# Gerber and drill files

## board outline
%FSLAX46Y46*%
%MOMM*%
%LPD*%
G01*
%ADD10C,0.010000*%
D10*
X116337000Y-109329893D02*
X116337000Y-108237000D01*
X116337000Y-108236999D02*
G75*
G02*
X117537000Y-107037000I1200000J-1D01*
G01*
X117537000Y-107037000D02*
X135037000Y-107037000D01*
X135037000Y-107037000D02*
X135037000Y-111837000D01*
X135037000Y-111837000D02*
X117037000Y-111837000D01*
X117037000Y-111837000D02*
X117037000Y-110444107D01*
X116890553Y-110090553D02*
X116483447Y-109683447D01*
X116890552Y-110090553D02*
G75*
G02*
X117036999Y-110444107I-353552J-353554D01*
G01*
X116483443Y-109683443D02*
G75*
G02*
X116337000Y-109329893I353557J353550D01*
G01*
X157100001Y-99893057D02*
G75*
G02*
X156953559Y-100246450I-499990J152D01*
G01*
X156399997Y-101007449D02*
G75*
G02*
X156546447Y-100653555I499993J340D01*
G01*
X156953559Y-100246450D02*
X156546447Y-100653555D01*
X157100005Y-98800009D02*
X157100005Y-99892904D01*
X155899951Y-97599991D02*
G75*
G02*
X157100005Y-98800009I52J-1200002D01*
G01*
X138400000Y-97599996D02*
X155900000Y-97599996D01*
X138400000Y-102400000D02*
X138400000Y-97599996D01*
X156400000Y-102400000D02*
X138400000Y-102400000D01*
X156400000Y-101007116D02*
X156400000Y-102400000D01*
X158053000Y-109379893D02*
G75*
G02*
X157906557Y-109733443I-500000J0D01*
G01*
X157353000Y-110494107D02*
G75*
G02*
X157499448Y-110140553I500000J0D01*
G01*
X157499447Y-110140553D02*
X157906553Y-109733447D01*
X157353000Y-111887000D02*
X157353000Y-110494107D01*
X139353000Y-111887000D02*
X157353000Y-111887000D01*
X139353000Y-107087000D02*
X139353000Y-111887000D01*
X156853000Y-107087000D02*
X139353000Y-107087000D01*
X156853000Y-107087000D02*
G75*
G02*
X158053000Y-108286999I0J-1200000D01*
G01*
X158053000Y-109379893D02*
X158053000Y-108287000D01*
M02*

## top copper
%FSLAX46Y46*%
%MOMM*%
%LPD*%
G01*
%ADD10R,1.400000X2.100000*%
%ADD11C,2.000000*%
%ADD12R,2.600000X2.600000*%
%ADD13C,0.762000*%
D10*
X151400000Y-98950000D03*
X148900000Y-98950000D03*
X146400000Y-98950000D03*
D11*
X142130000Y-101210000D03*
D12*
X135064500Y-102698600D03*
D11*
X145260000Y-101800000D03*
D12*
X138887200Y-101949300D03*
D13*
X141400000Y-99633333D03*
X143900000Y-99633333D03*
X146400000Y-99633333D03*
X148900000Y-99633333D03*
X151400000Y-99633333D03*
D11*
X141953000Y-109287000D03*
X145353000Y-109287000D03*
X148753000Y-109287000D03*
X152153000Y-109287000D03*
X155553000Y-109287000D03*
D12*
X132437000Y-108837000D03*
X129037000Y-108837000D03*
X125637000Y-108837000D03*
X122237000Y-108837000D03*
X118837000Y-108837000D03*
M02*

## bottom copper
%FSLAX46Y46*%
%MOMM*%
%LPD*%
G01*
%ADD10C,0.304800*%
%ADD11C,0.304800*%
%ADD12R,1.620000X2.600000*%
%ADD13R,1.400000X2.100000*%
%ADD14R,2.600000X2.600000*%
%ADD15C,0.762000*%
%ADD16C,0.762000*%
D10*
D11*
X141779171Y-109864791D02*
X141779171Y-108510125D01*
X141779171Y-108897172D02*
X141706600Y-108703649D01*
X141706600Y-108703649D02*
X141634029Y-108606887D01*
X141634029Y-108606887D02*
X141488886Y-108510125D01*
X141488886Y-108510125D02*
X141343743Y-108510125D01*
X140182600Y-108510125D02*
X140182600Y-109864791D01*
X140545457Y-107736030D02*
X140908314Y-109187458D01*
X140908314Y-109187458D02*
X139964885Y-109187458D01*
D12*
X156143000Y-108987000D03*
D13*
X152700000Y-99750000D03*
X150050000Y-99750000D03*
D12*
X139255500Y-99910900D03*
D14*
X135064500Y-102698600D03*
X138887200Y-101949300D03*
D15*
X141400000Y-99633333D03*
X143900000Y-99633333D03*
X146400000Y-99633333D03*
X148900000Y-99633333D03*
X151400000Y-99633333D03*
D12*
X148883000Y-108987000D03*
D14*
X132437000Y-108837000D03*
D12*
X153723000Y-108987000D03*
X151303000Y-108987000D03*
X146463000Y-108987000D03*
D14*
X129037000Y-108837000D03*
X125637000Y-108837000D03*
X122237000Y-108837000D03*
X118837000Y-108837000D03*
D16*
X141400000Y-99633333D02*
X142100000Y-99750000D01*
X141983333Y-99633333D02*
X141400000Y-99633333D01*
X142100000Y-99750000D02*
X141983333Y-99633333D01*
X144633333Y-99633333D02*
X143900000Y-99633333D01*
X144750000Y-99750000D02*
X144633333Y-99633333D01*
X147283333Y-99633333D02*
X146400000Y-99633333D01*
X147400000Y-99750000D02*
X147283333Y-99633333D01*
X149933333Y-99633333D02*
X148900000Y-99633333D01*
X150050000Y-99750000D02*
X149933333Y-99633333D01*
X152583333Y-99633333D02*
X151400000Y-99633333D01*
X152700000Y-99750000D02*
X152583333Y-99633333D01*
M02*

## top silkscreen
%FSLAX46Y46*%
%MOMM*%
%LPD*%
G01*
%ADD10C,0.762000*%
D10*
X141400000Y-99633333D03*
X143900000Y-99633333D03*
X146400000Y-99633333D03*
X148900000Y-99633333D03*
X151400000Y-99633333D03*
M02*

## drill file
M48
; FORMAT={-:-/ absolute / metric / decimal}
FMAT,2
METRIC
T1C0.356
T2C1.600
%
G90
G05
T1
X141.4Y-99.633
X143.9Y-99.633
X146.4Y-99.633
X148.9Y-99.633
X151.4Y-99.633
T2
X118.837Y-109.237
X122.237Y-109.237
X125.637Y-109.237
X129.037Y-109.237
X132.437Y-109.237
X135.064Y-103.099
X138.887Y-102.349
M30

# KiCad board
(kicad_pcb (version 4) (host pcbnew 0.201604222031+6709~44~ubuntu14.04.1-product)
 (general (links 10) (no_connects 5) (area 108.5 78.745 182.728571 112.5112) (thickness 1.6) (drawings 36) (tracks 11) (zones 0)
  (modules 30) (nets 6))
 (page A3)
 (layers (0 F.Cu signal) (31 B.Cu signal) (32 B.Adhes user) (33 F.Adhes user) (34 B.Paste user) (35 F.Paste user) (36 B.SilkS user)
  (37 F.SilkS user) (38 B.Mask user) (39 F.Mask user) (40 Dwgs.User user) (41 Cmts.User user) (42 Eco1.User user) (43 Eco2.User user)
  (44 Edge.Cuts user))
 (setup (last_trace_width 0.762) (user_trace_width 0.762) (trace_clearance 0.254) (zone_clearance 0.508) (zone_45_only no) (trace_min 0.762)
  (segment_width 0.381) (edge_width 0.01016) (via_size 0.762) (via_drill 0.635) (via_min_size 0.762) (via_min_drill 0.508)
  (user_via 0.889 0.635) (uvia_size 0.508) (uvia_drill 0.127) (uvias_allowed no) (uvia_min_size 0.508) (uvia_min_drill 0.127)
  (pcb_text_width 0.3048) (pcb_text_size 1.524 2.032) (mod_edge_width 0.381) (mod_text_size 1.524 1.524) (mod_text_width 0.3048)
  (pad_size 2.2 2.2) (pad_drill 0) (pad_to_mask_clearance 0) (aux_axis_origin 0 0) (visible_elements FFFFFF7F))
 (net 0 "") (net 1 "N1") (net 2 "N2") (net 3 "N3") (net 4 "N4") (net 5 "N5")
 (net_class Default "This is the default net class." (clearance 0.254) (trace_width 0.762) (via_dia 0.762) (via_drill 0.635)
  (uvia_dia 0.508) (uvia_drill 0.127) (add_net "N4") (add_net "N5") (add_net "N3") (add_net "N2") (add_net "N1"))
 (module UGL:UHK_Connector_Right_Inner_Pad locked (layer B.Cu) (at 156.143 108.987)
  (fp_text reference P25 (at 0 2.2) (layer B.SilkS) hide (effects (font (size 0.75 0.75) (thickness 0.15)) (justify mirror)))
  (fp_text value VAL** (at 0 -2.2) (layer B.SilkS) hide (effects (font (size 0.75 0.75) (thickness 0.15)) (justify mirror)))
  (pad "" smd rect (at 0 0) (size 1.62 2.6) (layers B.Cu B.Paste B.Mask)))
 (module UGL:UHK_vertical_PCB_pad (layer B.Cu) (at 152.7 99.75)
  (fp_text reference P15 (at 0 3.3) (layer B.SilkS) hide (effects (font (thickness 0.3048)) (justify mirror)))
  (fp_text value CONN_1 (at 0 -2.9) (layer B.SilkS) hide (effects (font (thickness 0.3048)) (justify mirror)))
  (pad "" smd rect (at 0 0) (size 1.4 2.1) (layers B.Cu B.Mask) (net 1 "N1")))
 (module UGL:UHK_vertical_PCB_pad (layer F.Cu) (at 151 98.95)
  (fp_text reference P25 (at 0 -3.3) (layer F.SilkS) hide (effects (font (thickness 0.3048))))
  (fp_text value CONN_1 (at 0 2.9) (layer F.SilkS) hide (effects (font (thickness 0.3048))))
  (pad "" smd rect (at 0.4 0) (size 1.4 2.1) (layers F.Cu F.Mask) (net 1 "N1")))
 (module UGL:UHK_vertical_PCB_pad (layer B.Cu) (at 150.05 99.75)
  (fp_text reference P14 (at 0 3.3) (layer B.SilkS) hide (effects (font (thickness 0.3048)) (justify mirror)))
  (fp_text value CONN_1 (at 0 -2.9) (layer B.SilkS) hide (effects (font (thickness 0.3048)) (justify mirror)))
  (pad "" smd rect (at 0 0) (size 1.4 2.1) (layers B.Cu B.Mask) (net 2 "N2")))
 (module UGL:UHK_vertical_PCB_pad (layer F.Cu) (at 148.5 98.95)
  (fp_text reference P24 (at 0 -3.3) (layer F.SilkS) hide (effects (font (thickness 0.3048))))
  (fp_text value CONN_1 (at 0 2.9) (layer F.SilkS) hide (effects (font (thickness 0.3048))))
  (pad "" smd rect (at 0.4 0) (size 1.4 2.1) (layers F.Cu F.Mask) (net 2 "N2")))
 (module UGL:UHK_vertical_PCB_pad (layer B.Cu) (at 139.2555 99.9109)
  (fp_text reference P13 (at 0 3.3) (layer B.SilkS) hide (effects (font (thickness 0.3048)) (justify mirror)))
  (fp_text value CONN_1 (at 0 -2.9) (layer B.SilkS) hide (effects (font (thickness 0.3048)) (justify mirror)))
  (pad "" smd rect (at 0 0) (size 1.62 2.6) (layers B.Cu B.Mask) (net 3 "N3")))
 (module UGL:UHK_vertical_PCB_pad (layer F.Cu) (at 146 98.95)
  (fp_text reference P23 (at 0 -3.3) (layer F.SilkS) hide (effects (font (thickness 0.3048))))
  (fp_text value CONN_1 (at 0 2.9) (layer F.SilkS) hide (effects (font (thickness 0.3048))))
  (pad "" smd rect (at 0.4 0) (size 1.4 2.1) (layers F.Cu F.Mask) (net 3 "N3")))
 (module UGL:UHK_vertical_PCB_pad (layer F.Cu) (at 141.73 101.21)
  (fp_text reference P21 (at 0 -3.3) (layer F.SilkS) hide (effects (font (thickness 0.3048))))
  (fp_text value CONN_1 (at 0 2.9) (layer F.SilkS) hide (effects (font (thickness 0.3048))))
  (pad "" smd circle (at 0.4 0) (size 2 2) (layers F.Cu F.Paste F.Mask) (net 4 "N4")))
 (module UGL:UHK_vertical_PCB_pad (layer B.Cu) (at 135.0645 103.0986)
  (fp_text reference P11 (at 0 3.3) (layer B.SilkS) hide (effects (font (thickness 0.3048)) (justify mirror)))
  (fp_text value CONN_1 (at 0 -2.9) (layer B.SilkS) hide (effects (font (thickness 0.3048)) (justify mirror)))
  (pad "" thru_hole rect (at 0 0) (size 2.6 2.6) (drill 1.6 (offset 0 -0.4)) (layers *.Cu *.Mask B.SilkS) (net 4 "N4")))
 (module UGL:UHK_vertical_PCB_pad (layer F.Cu) (at 144.86 101.8)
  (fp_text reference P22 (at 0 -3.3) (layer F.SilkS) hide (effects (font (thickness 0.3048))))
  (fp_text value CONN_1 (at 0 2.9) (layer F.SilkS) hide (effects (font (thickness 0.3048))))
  (pad "" smd circle (at 0.4 0) (size 2 2) (layers F.Cu F.Mask) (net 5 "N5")))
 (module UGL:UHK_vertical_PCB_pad (layer B.Cu) (at 138.8872 102.3493)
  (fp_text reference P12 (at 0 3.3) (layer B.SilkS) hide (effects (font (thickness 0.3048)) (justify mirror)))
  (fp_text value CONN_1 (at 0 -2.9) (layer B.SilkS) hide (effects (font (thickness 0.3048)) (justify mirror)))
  (pad "" thru_hole rect (at 0 0) (size 2.6 2.6) (drill 1.6 (offset 0 -0.4)) (layers *.Cu *.Mask B.SilkS) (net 5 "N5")))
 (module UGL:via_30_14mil (layer F.Cu) (at 141.4 99.633333)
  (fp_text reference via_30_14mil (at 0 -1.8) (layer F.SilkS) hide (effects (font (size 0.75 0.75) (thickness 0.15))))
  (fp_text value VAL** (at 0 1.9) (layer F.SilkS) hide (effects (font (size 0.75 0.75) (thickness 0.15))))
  (pad "" thru_hole circle (at 0 0) (size 0.762 0.762) (drill 0.3556) (layers *.Cu *.Mask F.SilkS) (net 4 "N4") (solder_mask_margin -1)))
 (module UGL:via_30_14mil (layer F.Cu) (at 143.9 99.633333)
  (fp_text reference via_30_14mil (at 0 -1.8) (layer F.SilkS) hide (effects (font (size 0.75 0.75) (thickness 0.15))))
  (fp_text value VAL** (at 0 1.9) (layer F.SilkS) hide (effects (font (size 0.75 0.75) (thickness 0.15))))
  (pad "" thru_hole circle (at 0 0) (size 0.762 0.762) (drill 0.3556) (layers *.Cu *.Mask F.SilkS) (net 5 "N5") (solder_mask_margin -1)))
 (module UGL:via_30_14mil (layer F.Cu) (at 146.4 99.633333)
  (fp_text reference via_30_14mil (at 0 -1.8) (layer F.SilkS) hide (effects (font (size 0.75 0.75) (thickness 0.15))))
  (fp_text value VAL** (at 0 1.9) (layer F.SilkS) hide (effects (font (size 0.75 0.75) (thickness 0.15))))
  (pad "" thru_hole circle (at 0 0) (size 0.762 0.762) (drill 0.3556) (layers *.Cu *.Mask F.SilkS) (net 3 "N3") (solder_mask_margin -1)))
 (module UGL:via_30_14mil (layer F.Cu) (at 148.9 99.633333)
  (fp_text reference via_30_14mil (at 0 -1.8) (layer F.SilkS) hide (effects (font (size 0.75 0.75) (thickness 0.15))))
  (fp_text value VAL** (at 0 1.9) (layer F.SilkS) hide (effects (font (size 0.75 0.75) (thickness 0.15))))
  (pad "" thru_hole circle (at 0 0) (size 0.762 0.762) (drill 0.3556) (layers *.Cu *.Mask F.SilkS) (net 2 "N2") (solder_mask_margin -1)))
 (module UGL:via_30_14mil (layer F.Cu) (at 151.4 99.633333)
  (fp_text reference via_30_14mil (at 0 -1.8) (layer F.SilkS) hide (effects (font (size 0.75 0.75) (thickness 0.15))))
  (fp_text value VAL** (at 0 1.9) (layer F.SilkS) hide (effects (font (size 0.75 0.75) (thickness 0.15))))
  (pad "" thru_hole circle (at 0 0) (size 0.762 0.762) (drill 0.3556) (layers *.Cu *.Mask F.SilkS) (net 1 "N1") (solder_mask_margin -1)))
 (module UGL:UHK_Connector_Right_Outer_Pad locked (layer F.Cu) (at 141.9352 109.2708)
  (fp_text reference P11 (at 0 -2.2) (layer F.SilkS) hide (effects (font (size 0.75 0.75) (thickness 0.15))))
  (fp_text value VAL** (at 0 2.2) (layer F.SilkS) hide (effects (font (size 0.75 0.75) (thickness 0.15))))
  (pad "" smd circle (at 0.0178 0.0162) (size 2 2) (layers F.Cu F.Mask)))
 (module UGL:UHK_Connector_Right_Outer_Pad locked (layer F.Cu) (at 145.4023 109.3343)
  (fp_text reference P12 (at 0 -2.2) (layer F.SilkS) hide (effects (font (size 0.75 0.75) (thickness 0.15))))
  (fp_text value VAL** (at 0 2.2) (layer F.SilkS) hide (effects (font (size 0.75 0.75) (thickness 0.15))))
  (pad "" smd circle (at -0.0493 -0.0473) (size 2 2) (layers F.Cu F.Mask)))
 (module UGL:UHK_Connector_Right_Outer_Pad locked (layer F.Cu) (at 148.6789 109.2708)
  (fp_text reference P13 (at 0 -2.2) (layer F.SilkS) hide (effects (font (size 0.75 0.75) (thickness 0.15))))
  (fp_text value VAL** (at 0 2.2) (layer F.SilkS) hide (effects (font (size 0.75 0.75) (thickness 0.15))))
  (pad "" smd circle (at 0.0741 0.0162) (size 2 2) (layers F.Cu F.Mask)))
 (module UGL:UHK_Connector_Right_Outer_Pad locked (layer F.Cu) (at 152.2476 109.3597)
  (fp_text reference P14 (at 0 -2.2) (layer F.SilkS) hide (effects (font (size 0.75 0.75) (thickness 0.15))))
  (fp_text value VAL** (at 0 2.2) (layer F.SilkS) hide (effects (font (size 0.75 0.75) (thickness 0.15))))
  (pad "" smd circle (at -0.0946 -0.0727) (size 2 2) (layers F.Cu F.Mask)))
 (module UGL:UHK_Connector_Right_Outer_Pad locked (layer F.Cu) (at 155.5496 109.22)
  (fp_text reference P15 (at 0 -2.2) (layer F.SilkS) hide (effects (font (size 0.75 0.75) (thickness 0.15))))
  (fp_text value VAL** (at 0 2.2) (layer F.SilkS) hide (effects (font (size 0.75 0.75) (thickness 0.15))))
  (pad "" smd circle (at 0.0034 0.067) (size 2 2) (layers F.Cu F.Mask)))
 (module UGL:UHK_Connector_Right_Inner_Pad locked (layer B.Cu) (at 148.883 108.987)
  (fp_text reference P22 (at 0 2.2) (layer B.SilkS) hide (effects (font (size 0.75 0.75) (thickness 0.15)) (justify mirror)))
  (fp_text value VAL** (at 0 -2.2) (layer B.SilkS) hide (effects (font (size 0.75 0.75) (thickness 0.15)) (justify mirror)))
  (pad "" smd rect (at 0 0) (size 1.62 2.6) (layers B.Cu B.Paste B.Mask)))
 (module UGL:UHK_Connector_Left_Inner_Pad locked (layer B.Cu) (at 132.437 109.237 180)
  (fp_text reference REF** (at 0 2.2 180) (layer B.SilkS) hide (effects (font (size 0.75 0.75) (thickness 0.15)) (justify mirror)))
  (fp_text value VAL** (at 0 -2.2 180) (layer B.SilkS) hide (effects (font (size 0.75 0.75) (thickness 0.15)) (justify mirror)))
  (pad "" thru_hole rect (at 0 0 180) (size 2.6 2.6) (drill 1.6 (offset 0 0.4)) (layers *.Cu *.Mask B.SilkS)))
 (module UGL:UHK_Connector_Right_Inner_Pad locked (layer B.Cu) (at 153.723 108.987)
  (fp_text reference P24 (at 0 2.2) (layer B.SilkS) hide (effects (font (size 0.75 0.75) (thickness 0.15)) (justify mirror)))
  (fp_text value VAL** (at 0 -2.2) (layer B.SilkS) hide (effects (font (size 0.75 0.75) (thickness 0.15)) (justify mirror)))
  (pad "" smd rect (at 0 0) (size 1.62 2.6) (layers B.Cu B.Paste B.Mask)))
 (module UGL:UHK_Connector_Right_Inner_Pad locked (layer B.Cu) (at 151.303 108.987)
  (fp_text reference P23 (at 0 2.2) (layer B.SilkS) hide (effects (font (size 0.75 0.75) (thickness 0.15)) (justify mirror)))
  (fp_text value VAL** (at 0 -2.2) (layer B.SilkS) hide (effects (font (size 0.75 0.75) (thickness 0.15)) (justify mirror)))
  (pad "" smd rect (at 0 0) (size 1.62 2.6) (layers B.Cu B.Paste B.Mask)))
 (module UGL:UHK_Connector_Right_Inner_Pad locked (layer B.Cu) (at 146.463 108.987)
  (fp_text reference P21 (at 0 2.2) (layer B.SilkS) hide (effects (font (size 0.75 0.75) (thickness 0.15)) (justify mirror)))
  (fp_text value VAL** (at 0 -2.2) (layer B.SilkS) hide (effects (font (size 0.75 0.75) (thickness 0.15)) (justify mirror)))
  (pad "" smd rect (at 0 0) (size 1.62 2.6) (layers B.Cu B.Paste B.Mask)))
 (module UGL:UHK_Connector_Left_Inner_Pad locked (layer B.Cu) (at 129.037 109.237 180)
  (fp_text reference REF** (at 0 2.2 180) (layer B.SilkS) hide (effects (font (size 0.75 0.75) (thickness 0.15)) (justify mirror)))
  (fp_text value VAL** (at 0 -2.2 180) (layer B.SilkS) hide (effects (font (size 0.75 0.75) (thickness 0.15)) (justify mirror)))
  (pad "" thru_hole rect (at 0 0 180) (size 2.6 2.6) (drill 1.6 (offset 0 0.4)) (layers *.Cu *.Mask B.SilkS)))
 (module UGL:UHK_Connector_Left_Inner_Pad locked (layer B.Cu) (at 125.637 109.237 180)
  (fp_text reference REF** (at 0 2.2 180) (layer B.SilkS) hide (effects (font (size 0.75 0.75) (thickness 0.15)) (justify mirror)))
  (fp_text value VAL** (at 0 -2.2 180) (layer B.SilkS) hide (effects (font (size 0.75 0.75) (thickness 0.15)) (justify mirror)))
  (pad "" thru_hole rect (at 0 0 180) (size 2.6 2.6) (drill 1.6 (offset 0 0.4)) (layers *.Cu *.Mask B.SilkS)))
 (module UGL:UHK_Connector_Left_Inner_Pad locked (layer B.Cu) (at 122.237 109.237 180)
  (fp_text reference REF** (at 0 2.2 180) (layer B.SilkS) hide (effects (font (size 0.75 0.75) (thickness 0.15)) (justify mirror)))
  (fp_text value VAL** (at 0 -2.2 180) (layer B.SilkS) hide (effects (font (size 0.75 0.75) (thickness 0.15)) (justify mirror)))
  (pad "" thru_hole rect (at 0 0 180) (size 2.6 2.6) (drill 1.6 (offset 0 0.4)) (layers *.Cu *.Mask B.SilkS)))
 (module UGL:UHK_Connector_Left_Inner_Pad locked (layer B.Cu) (at 118.837 109.237 180)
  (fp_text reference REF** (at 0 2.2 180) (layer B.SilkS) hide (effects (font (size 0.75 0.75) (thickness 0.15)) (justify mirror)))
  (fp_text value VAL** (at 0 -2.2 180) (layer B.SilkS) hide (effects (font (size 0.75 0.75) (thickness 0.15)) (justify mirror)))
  (pad "" thru_hole rect (at 0 0 180) (size 2.6 2.6) (drill 1.6 (offset 0 0.4)) (layers *.Cu *.Mask B.SilkS)))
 (gr_line (start 116.337 109.329893) (end 116.337 108.237) (angle 90) (layer Edge.Cuts) (width 0.01))
 (gr_arc (start 117.537 108.237) (end 117.537 107.037) (angle -89.99995347) (layer Edge.Cuts) (width 0.01))
 (gr_line (start 117.537 107.037) (end 135.037 107.037) (angle 90) (layer Edge.Cuts) (width 0.01))
 (gr_line (start 135.037 107.037) (end 135.037 111.837) (angle 90) (layer Edge.Cuts) (width 0.01))
 (gr_line (start 135.037 111.837) (end 117.037 111.837) (angle 90) (layer Edge.Cuts) (width 0.01))
 (gr_line (start 117.037 111.837) (end 117.037 110.444107) (angle 90) (layer Edge.Cuts) (width 0.01))
 (gr_line (start 116.890553 110.090553) (end 116.483447 109.683447) (angle 90) (layer Edge.Cuts) (width 0.01))
 (gr_arc (start 116.537 110.444107) (end 117.037 110.444107) (angle -45.00015451) (layer Edge.Cuts) (width 0.01))
 (gr_arc (start 116.837 109.329893) (end 116.337 109.329893) (angle -44.99944414) (layer Edge.Cuts) (width 0.01))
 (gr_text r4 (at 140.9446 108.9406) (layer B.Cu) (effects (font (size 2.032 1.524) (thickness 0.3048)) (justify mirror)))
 (gr_arc (start 156.600011 99.892905) (end 156.953559 100.24645) (angle -44.98236916) (layer Edge.Cuts) (width 0.01))
 (gr_arc (start 156.89999 101.007109) (end 156.546447 100.653555) (angle -45.03987133) (layer Edge.Cuts) (width 0.01))
 (gr_line (start 156.953559 100.24645) (end 156.546447 100.653555) (angle 90) (layer Edge.Cuts) (width 0.01))
 (gr_line (start 157.100005 98.800009) (end 157.100005 99.892904) (angle 90) (layer Edge.Cuts) (width 0.01))
 (gr_arc (start 155.900003 98.799993) (end 157.100005 98.800009) (angle -90.0032229) (layer Edge.Cuts) (width 0.01))
 (gr_line (start 138.4 97.599996) (end 155.9 97.599996) (angle 90) (layer Edge.Cuts) (width 0.01))
 (gr_line (start 138.4 102.4) (end 138.4 97.599996) (angle 90) (layer Edge.Cuts) (width 0.01))
 (gr_line (start 156.4 102.4) (end 138.4 102.4) (angle 90) (layer Edge.Cuts) (width 0.01))
 (gr_line (start 156.4 101.007116) (end 156.4 102.4) (angle 90) (layer Edge.Cuts) (width 0.01))
 (gr_arc (start 157.553 109.379893) (end 158.053 109.379893) (angle 44.99944414) (layer Edge.Cuts) (width 0.01))
 (gr_arc (start 157.853 110.494107) (end 157.353 110.494107) (angle 45.00015451) (layer Edge.Cuts) (width 0.01))
 (gr_line (start 157.499447 110.140553) (end 157.906553 109.733447) (angle 90) (layer Edge.Cuts) (width 0.01))
 (gr_line (start 157.353 111.887) (end 157.353 110.494107) (angle 90) (layer Edge.Cuts) (width 0.01))
 (gr_line (start 139.353 111.887) (end 157.353 111.887) (angle 90) (layer Edge.Cuts) (width 0.01))
 (gr_line (start 139.353 107.087) (end 139.353 111.887) (angle 90) (layer Edge.Cuts) (width 0.01))
 (gr_line (start 156.853 107.087) (end 139.353 107.087) (angle 90) (layer Edge.Cuts) (width 0.01))
 (gr_arc (start 156.853 108.287) (end 156.853 107.087) (angle 89.99995347) (layer Edge.Cuts) (width 0.01))
 (gr_line (start 158.053 109.379893) (end 158.053 108.287) (angle 90) (layer Edge.Cuts) (width 0.01))
 (segment (start 141.4 99.633333) (end 142.1 99.75) (width 0.762) (layer B.Cu) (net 4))
 (segment (start 141.983333 99.633333) (end 141.4 99.633333) (width 0.762) (layer B.Cu) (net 4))
 (segment (start 142.1 99.75) (end 141.983333 99.633333) (width 0.762) (layer B.Cu) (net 4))
 (segment (start 144.633333 99.633333) (end 143.9 99.633333) (width 0.762) (layer B.Cu) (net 5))
 (segment (start 144.75 99.75) (end 144.633333 99.633333) (width 0.762) (layer B.Cu) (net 5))
 (segment (start 147.283333 99.633333) (end 146.4 99.633333) (width 0.762) (layer B.Cu) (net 3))
 (segment (start 147.4 99.75) (end 147.283333 99.633333) (width 0.762) (layer B.Cu) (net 3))
 (segment (start 149.933333 99.633333) (end 148.9 99.633333) (width 0.762) (layer B.Cu) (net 2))
 (segment (start 150.05 99.75) (end 149.933333 99.633333) (width 0.762) (layer B.Cu) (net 2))
 (segment (start 152.583333 99.633333) (end 151.4 99.633333) (width 0.762) (layer B.Cu) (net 1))
 (segment (start 152.7 99.75) (end 152.583333 99.633333) (width 0.762) (layer B.Cu) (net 1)))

